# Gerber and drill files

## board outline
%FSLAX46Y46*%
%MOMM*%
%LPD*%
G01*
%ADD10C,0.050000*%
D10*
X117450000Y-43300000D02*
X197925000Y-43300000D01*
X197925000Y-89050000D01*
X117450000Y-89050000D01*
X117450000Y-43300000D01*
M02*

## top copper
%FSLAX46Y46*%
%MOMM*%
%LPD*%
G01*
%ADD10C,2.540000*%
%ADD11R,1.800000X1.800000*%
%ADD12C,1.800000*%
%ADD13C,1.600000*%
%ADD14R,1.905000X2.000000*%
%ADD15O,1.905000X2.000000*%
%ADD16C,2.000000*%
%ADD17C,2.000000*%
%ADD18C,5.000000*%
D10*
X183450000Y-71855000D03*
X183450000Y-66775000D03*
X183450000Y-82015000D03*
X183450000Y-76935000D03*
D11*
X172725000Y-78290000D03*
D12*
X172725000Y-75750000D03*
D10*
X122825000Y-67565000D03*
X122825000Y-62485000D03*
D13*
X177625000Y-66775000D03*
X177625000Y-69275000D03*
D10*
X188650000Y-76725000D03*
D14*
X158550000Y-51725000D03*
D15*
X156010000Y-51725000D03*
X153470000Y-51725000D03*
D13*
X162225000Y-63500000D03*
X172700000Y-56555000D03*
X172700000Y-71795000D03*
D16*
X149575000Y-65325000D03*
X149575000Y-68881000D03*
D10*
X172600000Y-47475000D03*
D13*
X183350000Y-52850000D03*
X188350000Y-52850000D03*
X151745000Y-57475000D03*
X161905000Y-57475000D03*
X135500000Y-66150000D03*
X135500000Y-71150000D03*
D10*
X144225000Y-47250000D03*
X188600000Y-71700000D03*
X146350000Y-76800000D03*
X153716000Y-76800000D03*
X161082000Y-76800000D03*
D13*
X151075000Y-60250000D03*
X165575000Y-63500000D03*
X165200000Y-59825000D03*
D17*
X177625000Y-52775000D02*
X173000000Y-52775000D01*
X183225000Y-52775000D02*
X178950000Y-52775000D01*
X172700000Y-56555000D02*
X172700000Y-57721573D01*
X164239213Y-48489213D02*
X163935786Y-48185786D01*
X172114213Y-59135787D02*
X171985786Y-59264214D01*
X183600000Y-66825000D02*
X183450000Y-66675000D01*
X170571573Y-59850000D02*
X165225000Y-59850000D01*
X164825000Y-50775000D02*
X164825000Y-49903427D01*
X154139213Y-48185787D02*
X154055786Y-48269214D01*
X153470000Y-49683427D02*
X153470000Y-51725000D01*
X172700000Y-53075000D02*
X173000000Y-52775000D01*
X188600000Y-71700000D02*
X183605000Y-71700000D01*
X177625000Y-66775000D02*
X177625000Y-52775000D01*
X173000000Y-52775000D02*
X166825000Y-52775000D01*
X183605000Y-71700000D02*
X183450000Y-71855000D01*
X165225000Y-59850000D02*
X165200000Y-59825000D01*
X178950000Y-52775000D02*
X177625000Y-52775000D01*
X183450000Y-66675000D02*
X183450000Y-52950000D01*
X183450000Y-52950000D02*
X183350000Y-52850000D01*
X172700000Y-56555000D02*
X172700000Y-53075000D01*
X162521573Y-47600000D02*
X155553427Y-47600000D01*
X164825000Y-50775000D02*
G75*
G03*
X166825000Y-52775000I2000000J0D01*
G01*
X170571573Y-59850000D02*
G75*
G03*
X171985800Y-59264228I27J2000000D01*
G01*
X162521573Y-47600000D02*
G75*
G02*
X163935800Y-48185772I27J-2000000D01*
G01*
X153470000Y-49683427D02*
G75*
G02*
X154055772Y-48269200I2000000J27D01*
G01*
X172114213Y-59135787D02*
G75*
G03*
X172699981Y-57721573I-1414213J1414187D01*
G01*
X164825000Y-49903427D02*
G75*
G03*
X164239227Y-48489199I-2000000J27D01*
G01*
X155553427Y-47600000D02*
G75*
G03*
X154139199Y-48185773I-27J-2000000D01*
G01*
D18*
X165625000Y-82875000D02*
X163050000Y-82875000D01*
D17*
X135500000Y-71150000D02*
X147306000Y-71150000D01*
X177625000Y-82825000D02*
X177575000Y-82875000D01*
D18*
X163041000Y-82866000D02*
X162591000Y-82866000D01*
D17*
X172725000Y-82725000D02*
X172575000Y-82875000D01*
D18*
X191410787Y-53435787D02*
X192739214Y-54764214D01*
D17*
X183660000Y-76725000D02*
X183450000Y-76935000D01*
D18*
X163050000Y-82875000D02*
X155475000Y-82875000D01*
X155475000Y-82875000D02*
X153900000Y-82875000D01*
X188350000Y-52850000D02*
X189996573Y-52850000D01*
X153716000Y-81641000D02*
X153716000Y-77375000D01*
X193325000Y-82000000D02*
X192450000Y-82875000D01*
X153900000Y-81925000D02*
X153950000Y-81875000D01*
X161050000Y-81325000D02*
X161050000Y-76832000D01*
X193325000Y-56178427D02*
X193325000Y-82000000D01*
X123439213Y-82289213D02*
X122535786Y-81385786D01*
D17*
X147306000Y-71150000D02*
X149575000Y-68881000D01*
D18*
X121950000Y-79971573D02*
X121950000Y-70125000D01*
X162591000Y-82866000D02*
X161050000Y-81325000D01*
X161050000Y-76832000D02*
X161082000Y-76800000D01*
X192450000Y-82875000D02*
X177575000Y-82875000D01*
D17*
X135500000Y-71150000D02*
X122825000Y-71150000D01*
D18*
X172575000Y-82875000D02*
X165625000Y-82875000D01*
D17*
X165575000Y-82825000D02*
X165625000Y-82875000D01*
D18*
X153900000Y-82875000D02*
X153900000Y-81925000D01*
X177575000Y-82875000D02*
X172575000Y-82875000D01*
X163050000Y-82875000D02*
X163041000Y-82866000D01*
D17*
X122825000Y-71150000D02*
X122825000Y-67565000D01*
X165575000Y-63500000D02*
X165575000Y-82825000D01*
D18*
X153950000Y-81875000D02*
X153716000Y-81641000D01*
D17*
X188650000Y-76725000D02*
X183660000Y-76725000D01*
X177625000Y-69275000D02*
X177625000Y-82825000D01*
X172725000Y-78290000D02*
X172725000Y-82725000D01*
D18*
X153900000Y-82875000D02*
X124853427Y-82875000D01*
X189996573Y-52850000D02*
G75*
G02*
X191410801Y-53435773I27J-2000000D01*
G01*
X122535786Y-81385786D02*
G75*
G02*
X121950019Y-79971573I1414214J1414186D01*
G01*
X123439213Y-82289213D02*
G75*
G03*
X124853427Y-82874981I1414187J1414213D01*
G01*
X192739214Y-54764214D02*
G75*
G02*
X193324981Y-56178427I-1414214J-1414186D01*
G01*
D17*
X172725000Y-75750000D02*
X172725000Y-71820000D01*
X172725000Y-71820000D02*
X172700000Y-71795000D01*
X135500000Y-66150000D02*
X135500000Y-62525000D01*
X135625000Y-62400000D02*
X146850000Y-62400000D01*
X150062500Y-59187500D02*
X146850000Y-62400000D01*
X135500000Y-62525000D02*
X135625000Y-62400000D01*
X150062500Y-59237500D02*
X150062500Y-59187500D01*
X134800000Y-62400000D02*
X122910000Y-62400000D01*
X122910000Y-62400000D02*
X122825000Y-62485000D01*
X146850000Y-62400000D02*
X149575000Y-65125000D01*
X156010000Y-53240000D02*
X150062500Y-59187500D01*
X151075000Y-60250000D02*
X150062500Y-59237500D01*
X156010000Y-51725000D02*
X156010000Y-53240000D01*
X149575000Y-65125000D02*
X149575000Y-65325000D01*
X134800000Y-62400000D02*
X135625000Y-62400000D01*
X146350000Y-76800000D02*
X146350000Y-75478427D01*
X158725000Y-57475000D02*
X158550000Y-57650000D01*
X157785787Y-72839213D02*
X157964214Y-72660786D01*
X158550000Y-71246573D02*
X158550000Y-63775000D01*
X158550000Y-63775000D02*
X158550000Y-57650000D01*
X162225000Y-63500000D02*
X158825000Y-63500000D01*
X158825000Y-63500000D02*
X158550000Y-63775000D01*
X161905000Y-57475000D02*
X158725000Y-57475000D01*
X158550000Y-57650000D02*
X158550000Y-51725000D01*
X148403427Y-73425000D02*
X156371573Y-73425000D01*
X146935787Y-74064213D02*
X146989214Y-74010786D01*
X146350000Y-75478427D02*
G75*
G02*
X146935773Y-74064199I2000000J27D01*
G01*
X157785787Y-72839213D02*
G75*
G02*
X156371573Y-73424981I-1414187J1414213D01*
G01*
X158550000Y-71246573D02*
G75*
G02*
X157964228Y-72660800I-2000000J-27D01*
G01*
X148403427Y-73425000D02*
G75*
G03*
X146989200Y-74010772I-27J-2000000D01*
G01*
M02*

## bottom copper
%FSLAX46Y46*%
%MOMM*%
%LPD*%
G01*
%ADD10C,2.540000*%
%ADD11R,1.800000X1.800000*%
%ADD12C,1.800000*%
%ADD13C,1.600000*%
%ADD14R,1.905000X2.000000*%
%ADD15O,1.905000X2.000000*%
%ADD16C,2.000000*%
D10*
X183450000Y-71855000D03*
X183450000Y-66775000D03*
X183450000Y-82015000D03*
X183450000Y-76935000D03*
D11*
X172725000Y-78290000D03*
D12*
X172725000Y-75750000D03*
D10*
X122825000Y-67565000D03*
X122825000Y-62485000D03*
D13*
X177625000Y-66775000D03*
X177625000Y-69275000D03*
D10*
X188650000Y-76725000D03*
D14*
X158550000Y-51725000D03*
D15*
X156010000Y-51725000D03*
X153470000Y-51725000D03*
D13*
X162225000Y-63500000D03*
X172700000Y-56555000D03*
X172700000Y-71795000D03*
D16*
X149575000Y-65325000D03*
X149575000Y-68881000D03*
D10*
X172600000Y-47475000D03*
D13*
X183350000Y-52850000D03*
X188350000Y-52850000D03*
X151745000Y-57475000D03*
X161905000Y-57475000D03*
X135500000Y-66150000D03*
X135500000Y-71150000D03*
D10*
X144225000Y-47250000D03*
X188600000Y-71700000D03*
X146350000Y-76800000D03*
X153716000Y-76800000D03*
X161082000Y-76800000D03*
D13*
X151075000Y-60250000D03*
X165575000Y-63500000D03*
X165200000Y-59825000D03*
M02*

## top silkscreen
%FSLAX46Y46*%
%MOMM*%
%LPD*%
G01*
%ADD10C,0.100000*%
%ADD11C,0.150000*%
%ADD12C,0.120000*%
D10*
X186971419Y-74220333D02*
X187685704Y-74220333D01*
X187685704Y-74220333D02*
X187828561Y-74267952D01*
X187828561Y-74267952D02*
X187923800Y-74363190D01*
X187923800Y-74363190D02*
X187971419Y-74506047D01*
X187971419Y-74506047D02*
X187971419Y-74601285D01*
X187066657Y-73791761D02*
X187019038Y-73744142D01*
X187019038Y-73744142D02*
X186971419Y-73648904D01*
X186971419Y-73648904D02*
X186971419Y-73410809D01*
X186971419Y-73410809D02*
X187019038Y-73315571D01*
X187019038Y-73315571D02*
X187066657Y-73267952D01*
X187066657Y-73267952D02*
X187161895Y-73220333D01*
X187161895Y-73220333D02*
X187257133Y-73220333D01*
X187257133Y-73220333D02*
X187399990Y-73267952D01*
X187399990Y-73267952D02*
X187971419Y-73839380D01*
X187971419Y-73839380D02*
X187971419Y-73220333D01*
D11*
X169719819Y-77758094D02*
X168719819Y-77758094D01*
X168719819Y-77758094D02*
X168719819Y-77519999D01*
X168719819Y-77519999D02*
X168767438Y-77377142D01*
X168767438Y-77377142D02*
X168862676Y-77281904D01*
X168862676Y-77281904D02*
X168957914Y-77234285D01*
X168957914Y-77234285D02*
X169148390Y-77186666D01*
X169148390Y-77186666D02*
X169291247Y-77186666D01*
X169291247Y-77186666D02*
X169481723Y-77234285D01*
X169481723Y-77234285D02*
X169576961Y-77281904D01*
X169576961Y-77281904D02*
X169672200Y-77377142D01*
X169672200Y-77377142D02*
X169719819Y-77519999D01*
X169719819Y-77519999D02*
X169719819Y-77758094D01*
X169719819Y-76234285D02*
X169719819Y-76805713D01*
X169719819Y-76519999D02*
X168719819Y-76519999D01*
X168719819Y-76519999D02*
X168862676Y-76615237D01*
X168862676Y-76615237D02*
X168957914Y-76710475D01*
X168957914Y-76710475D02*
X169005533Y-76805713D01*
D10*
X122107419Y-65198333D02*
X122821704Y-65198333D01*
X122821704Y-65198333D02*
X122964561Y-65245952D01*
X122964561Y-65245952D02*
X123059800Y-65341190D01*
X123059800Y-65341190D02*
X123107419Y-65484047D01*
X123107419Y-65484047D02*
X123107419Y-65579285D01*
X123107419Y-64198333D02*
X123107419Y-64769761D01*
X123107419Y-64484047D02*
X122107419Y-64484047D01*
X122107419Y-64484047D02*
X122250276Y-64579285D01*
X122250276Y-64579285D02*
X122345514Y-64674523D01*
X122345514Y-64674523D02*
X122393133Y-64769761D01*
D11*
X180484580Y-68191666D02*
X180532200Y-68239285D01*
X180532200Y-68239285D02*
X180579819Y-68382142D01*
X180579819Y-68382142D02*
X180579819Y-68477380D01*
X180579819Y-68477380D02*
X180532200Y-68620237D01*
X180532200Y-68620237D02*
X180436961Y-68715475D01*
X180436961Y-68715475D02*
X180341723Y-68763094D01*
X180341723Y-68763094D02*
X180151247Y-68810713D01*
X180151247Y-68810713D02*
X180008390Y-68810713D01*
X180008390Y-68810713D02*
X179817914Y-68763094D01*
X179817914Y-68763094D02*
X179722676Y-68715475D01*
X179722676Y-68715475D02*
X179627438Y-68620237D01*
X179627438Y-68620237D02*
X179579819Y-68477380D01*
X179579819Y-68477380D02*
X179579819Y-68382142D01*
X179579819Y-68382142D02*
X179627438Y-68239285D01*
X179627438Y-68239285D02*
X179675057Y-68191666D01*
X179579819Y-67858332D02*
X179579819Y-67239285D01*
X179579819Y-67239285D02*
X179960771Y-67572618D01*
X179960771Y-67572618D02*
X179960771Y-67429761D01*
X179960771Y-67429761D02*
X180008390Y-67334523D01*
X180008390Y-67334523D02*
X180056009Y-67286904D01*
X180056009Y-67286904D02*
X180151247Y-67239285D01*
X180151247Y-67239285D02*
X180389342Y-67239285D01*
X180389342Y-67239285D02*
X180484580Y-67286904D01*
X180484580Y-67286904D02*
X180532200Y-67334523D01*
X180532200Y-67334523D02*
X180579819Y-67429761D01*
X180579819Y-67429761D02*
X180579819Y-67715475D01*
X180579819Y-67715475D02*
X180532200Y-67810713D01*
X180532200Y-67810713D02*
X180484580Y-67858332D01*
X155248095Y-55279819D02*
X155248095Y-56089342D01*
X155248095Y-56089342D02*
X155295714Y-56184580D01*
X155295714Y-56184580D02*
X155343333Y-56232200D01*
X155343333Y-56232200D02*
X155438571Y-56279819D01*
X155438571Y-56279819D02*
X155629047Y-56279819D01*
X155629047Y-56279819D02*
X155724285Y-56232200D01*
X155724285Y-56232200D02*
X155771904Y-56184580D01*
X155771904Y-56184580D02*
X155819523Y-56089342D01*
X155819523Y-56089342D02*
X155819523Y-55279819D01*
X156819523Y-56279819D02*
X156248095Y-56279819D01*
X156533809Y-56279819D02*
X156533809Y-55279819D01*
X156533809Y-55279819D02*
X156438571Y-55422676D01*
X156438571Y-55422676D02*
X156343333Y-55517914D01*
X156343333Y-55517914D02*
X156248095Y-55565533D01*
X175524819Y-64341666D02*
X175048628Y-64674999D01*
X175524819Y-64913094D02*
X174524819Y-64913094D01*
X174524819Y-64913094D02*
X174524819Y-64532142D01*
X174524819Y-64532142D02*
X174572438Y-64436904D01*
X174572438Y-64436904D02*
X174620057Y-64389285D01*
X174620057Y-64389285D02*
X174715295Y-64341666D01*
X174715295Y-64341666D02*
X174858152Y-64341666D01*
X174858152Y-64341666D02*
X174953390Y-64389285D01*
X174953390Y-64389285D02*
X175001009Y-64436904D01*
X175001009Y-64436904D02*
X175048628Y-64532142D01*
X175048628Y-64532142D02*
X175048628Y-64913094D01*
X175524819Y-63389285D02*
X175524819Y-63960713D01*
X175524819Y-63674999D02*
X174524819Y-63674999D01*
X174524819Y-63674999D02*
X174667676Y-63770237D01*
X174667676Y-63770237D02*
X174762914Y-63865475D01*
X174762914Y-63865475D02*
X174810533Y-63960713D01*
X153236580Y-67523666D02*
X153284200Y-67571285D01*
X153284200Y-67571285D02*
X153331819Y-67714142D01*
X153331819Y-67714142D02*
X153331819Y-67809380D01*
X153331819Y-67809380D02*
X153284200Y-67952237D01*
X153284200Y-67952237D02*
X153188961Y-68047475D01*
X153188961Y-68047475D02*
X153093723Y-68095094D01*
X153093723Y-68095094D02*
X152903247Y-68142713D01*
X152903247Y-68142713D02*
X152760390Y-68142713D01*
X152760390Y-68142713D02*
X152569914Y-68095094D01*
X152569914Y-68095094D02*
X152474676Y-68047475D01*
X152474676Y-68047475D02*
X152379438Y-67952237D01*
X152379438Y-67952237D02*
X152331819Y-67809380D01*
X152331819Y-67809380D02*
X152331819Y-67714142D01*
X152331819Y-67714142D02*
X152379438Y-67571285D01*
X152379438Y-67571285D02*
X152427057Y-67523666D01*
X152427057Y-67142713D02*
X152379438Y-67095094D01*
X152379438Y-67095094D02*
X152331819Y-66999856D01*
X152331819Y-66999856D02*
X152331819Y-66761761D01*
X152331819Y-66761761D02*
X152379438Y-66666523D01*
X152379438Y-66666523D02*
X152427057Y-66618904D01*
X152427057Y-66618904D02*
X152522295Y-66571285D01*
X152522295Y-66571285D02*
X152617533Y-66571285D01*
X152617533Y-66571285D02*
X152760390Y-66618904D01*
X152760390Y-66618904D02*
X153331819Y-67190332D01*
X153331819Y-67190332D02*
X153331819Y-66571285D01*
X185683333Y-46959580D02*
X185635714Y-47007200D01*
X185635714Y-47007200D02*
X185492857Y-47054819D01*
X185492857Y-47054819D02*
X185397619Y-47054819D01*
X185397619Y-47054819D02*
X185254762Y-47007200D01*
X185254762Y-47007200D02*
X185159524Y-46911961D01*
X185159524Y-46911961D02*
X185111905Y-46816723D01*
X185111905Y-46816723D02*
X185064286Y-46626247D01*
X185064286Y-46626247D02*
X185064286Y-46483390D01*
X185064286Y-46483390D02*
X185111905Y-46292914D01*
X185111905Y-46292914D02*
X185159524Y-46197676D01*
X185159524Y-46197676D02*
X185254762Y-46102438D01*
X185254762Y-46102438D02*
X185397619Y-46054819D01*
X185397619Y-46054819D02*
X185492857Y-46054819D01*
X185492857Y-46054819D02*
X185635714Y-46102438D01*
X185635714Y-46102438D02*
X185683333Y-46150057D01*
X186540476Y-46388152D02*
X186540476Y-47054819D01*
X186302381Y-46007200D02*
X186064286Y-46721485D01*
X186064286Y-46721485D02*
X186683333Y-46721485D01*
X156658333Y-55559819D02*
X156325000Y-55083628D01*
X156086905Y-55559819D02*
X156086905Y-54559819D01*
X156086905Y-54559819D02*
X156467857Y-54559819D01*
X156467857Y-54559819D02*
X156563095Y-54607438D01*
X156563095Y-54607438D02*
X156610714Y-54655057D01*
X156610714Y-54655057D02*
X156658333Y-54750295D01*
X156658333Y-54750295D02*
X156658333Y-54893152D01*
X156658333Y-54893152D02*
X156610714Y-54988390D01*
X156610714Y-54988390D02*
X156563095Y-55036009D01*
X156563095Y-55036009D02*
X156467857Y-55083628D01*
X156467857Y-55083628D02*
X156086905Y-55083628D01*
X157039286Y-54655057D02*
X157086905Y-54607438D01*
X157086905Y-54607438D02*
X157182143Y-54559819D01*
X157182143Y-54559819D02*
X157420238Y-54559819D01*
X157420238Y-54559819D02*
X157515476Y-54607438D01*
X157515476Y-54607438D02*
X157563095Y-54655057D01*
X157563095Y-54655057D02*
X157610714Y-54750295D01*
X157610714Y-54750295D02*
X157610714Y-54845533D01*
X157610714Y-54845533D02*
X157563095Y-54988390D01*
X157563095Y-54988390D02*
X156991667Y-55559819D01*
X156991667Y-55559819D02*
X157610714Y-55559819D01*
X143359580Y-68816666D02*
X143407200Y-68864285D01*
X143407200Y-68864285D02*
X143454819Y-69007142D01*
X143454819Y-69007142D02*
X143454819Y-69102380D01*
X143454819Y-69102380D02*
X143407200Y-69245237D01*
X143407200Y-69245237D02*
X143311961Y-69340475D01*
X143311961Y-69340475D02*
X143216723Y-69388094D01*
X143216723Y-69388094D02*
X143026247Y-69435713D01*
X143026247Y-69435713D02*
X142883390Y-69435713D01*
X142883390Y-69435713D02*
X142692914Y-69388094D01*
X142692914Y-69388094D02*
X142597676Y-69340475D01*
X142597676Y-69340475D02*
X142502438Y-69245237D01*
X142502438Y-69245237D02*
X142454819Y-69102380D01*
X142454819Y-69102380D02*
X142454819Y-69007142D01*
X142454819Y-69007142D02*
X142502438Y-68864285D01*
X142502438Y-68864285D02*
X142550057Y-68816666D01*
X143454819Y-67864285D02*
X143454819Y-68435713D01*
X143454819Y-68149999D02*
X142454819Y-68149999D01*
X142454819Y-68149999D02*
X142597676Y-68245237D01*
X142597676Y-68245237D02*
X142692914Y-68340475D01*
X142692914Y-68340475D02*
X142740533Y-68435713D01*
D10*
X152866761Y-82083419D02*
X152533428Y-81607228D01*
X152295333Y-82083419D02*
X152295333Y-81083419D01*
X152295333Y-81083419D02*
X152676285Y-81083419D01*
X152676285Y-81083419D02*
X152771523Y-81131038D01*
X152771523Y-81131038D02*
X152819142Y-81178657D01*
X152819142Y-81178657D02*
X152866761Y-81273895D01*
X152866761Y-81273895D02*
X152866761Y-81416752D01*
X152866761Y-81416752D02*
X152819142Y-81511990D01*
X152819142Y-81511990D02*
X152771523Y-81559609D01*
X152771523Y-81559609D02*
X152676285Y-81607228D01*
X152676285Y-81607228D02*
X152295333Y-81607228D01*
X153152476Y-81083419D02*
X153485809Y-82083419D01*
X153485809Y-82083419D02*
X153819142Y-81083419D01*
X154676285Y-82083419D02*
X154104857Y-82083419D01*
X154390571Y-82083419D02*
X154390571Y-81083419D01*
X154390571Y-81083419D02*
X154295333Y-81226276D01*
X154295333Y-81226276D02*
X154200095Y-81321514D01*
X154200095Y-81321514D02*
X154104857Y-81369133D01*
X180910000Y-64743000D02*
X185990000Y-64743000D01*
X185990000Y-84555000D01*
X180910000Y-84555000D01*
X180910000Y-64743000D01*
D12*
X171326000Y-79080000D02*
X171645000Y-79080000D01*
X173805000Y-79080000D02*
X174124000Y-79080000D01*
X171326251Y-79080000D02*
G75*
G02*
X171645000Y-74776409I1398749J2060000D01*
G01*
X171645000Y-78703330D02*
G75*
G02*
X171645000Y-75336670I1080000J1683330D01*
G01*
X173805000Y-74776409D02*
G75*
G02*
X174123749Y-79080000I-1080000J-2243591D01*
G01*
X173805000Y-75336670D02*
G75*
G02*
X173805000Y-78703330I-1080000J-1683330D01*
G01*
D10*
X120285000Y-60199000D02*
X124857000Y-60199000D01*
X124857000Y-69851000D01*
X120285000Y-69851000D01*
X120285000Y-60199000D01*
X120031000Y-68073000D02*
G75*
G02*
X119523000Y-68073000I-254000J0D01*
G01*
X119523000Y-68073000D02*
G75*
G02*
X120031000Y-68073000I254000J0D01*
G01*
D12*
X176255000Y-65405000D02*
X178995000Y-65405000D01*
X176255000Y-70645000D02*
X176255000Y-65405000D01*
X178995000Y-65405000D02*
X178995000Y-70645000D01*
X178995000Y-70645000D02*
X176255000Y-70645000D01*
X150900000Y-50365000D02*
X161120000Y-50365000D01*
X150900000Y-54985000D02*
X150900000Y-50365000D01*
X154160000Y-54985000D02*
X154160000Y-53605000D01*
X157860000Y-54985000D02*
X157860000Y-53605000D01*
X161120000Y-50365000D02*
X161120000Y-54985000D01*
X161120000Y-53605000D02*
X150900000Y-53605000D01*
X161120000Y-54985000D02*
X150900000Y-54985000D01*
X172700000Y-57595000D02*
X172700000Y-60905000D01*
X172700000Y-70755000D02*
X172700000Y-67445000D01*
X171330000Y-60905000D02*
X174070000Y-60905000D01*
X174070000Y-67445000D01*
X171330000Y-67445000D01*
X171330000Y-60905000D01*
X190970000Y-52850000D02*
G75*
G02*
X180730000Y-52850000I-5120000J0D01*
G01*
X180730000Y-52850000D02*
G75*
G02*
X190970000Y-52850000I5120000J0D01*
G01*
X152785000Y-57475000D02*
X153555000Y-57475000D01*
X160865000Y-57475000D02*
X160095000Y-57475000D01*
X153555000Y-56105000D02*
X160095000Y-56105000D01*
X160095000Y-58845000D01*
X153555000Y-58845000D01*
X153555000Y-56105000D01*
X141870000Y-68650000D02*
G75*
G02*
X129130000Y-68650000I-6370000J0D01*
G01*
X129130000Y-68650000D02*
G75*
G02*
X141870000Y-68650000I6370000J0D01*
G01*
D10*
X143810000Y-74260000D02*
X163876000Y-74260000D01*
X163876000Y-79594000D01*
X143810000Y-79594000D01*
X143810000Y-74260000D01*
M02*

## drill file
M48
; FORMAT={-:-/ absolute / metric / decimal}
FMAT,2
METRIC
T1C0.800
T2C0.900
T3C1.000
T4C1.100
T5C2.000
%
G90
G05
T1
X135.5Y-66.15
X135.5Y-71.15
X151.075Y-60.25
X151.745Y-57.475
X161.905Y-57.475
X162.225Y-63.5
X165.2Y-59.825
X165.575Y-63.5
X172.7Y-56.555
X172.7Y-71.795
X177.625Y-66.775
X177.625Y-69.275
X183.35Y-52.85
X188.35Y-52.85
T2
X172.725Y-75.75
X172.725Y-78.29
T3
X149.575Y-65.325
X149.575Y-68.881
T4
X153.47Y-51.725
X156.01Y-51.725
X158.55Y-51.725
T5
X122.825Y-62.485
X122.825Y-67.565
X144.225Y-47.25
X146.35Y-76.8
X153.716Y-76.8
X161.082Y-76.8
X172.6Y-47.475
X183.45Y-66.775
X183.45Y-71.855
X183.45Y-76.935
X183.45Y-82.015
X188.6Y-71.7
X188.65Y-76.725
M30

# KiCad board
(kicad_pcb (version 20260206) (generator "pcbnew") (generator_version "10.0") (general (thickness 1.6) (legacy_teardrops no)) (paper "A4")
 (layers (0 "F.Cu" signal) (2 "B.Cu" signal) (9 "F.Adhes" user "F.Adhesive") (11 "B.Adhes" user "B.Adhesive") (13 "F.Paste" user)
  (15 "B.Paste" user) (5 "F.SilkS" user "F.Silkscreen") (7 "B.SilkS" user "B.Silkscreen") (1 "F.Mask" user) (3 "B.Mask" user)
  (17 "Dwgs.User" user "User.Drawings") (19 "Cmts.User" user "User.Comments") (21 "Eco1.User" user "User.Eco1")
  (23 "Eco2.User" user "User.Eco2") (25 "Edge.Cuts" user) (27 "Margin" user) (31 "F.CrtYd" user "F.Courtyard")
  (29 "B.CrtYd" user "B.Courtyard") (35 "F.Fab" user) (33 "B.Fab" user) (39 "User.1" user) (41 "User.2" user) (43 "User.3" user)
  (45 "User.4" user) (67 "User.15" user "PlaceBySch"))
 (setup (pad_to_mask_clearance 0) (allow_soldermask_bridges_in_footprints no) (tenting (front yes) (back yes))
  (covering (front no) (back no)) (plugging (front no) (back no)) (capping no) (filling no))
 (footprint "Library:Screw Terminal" (layer "F.Cu") (at 183.45 74.395 90)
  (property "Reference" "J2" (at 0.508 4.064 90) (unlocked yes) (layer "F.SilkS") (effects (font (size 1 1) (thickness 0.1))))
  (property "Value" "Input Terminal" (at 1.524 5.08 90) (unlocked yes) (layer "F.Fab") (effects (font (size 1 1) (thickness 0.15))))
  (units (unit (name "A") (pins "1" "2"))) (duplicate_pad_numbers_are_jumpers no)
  (fp_rect (start -10.16 -2.54) (end 9.652 2.54) (stroke (width 0.1) (type default)) (fill no) (layer "F.SilkS"))
  (pad "1" thru_hole circle (at 2.54 0 90) (size 2.54 2.54) (drill 2) (layers "*.Cu" "*.Mask") (remove_unused_layers no)
   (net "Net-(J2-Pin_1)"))
  (pad "1" thru_hole circle (at 7.62 0 90) (size 2.54 2.54) (drill 2) (layers "*.Cu" "*.Mask") (remove_unused_layers no)
   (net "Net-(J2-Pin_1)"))
  (pad "2" thru_hole circle (at -7.62 0 90) (size 2.54 2.54) (drill 2) (layers "*.Cu" "*.Mask") (remove_unused_layers no) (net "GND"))
  (pad "2" thru_hole circle (at -2.54 0 90) (size 2.54 2.54) (drill 2) (layers "*.Cu" "*.Mask") (remove_unused_layers no) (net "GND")))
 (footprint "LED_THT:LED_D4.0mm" (layer "F.Cu") (at 172.725 78.29 90)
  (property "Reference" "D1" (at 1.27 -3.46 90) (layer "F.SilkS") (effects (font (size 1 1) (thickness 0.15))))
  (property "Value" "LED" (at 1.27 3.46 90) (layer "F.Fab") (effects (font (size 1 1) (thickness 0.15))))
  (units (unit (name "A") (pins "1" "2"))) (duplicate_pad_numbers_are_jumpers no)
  (fp_line (start -0.79 -1.399) (end -0.79 -1.08) (stroke (width 0.12) (type solid)) (layer "F.SilkS"))
  (fp_line (start -0.79 1.08) (end -0.79 1.399) (stroke (width 0.12) (type solid)) (layer "F.SilkS"))
  (fp_arc (start -0.79 -1.398749) (mid 1.45392 -2.483198) (end 3.513591 -1.08) (stroke (width 0.12) (type solid)) (layer "F.SilkS"))
  (fp_arc (start -0.41333 -1.08) (mid 1.27 -2) (end 2.95333 -1.08) (stroke (width 0.12) (type solid)) (layer "F.SilkS"))
  (fp_arc (start 3.513591 1.08) (mid 1.45392 2.483198) (end -0.79 1.398749) (stroke (width 0.12) (type solid)) (layer "F.SilkS"))
  (fp_arc (start 2.95333 1.08) (mid 1.27 2) (end -0.41333 1.08) (stroke (width 0.12) (type solid)) (layer "F.SilkS"))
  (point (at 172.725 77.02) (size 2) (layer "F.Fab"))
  (pad "1" thru_hole rect (at 0 0 90) (size 1.8 1.8) (drill 0.9) (layers "*.Cu" "*.Mask") (remove_unused_layers no) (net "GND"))
  (pad "2" thru_hole circle (at 2.54 0 90) (size 1.8 1.8) (drill 0.9) (layers "*.Cu" "*.Mask") (remove_unused_layers no) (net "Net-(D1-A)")))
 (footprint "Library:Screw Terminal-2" (layer "F.Cu") (at 122.825 65.025 90)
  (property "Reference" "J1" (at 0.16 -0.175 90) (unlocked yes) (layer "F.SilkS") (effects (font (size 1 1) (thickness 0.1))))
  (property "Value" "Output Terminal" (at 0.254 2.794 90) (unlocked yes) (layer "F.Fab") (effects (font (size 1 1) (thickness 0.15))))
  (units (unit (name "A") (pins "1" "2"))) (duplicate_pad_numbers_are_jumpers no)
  (fp_rect (start -4.826 -2.54) (end 4.826 2.032) (stroke (width 0.1) (type default)) (fill no) (layer "F.SilkS"))
  (fp_circle (center -3.048 -3.048) (end -2.794 -3.048) (stroke (width 0.1) (type solid)) (fill no) (layer "F.SilkS"))
  (pad "1" thru_hole circle (at -2.54 0 90) (size 2.54 2.54) (drill 2) (layers "*.Cu" "*.Mask") (remove_unused_layers no) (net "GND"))
  (pad "2" thru_hole circle (at 2.54 0 180) (size 2.54 2.54) (drill 2) (layers "*.Cu" "*.Mask") (remove_unused_layers no)
   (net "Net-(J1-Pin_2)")))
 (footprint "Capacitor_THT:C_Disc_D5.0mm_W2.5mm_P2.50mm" (layer "F.Cu") (at 177.625 66.775 -90)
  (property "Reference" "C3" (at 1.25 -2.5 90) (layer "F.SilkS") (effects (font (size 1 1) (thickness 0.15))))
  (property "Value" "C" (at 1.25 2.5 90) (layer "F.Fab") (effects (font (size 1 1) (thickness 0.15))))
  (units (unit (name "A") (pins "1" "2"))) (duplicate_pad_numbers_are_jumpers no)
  (fp_line (start -1.37 1.37) (end -1.37 -1.37) (stroke (width 0.12) (type solid)) (layer "F.SilkS"))
  (fp_line (start 3.87 1.37) (end -1.37 1.37) (stroke (width 0.12) (type solid)) (layer "F.SilkS"))
  (fp_line (start -1.37 -1.37) (end 3.87 -1.37) (stroke (width 0.12) (type solid)) (layer "F.SilkS"))
  (fp_line (start 3.87 -1.37) (end 3.87 1.37) (stroke (width 0.12) (type solid)) (layer "F.SilkS"))
  (pad "1" thru_hole circle (at 0 0 270) (size 1.6 1.6) (drill 0.8) (layers "*.Cu" "*.Mask") (remove_unused_layers no)
   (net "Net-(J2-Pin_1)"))
  (pad "2" thru_hole circle (at 2.5 0 270) (size 1.6 1.6) (drill 0.8) (layers "*.Cu" "*.Mask") (remove_unused_layers no) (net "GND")))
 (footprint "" (layer "F.Cu") (at 188.65 76.725)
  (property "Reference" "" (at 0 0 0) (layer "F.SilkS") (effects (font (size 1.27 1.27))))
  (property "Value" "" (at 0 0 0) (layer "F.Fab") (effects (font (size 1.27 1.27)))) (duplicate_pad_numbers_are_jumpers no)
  (pad "2" thru_hole circle (at 0 0 90) (size 2.54 2.54) (drill 2) (layers "*.Cu" "*.Mask") (remove_unused_layers no) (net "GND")))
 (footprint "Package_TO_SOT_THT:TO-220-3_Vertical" (layer "F.Cu") (at 158.55 51.725 180)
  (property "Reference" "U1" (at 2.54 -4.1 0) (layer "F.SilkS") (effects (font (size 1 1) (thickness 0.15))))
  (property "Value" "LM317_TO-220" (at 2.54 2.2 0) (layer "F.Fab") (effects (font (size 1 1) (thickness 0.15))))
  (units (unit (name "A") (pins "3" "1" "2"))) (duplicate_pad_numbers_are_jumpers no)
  (fp_line (start 7.65 1.36) (end -2.57 1.36) (stroke (width 0.12) (type solid)) (layer "F.SilkS"))
  (fp_line (start 7.65 -3.26) (end 7.65 1.36) (stroke (width 0.12) (type solid)) (layer "F.SilkS"))
  (fp_line (start 4.39 -3.26) (end 4.39 -1.88) (stroke (width 0.12) (type solid)) (layer "F.SilkS"))
  (fp_line (start 0.69 -3.26) (end 0.69 -1.88) (stroke (width 0.12) (type solid)) (layer "F.SilkS"))
  (fp_line (start -2.57 1.36) (end -2.57 -3.26) (stroke (width 0.12) (type solid)) (layer "F.SilkS"))
  (fp_line (start -2.57 -1.88) (end 7.65 -1.88) (stroke (width 0.12) (type solid)) (layer "F.SilkS"))
  (fp_line (start -2.57 -3.26) (end 7.65 -3.26) (stroke (width 0.12) (type solid)) (layer "F.SilkS"))
  (pad "1" thru_hole rect (at 0 0 180) (size 1.905 2) (drill 1.1) (layers "*.Cu" "*.Mask") (remove_unused_layers no) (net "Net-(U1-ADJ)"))
  (pad "2" thru_hole oval (at 2.54 0 180) (size 1.905 2) (drill 1.1) (layers "*.Cu" "*.Mask") (remove_unused_layers no)
   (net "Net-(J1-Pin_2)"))
  (pad "3" thru_hole oval (at 5.08 0 180) (size 1.905 2) (drill 1.1) (layers "*.Cu" "*.Mask") (remove_unused_layers no)
   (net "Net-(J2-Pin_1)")))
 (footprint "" (layer "F.Cu") (at 162.225 63.5)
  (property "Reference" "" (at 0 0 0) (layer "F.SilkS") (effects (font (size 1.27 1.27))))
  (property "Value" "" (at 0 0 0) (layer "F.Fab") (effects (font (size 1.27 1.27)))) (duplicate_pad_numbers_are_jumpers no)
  (pad "2" thru_hole circle (at 0 0) (size 1.6 1.6) (drill 0.8) (layers "*.Cu" "*.Mask") (remove_unused_layers no) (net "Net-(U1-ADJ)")))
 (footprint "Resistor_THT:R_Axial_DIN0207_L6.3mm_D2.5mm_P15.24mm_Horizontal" (layer "F.Cu") (at 172.7 56.555 -90)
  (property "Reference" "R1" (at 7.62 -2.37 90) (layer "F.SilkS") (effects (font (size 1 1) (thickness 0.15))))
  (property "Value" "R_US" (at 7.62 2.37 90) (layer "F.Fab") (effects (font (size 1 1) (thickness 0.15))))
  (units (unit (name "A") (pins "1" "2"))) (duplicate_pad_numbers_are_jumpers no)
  (fp_line (start 1.04 0) (end 4.35 0) (stroke (width 0.12) (type solid)) (layer "F.SilkS"))
  (fp_line (start 14.2 0) (end 10.89 0) (stroke (width 0.12) (type solid)) (layer "F.SilkS"))
  (fp_rect (start 4.35 -1.37) (end 10.89 1.37) (stroke (width 0.12) (type solid)) (fill no) (layer "F.SilkS"))
  (pad "1" thru_hole circle (at 0 0 270) (size 1.6 1.6) (drill 0.8) (layers "*.Cu" "*.Mask") (remove_unused_layers no)
   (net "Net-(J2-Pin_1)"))
  (pad "2" thru_hole circle (at 15.24 0 270) (size 1.6 1.6) (drill 0.8) (layers "*.Cu" "*.Mask") (remove_unused_layers no)
   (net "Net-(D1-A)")))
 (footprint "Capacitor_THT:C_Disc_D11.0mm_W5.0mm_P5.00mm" (layer "F.Cu") (at 149.575 65.325 -90)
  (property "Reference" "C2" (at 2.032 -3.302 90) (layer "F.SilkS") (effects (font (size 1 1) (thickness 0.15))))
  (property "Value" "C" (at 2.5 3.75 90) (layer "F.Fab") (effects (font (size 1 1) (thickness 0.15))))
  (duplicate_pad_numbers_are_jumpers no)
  (pad "1" thru_hole circle (at 0 0 270) (size 2 2) (drill 1) (layers "*.Cu" "*.Mask") (remove_unused_layers no) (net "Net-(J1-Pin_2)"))
  (pad "2" thru_hole circle (at 3.556 0 270) (size 2 2) (drill 1) (layers "*.Cu" "*.Mask") (remove_unused_layers no) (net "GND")))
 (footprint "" (layer "F.Cu") (at 172.6 47.475)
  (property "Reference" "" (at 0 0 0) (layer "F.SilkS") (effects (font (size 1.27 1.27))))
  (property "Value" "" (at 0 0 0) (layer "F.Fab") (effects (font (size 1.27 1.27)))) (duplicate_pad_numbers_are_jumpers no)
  (pad "3" thru_hole circle (at 0 0) (size 2.54 2.54) (drill 2) (layers "*.Cu" "*.Mask") (remove_unused_layers no) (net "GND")))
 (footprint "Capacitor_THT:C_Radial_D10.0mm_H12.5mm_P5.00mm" (layer "F.Cu") (at 183.35 52.85)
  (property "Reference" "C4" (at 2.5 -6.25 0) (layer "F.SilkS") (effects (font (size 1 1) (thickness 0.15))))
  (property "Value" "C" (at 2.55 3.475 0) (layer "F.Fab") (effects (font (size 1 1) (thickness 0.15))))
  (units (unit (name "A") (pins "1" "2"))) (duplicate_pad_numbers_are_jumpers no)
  (fp_circle (center 2.5 0) (end 7.62 0) (stroke (width 0.12) (type solid)) (fill no) (layer "F.SilkS"))
  (pad "1" thru_hole circle (at 0 0) (size 1.6 1.6) (drill 0.8) (layers "*.Cu" "*.Mask") (remove_unused_layers no) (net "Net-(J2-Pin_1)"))
  (pad "2" thru_hole circle (at 5 0) (size 1.6 1.6) (drill 0.8) (layers "*.Cu" "*.Mask") (remove_unused_layers no) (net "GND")))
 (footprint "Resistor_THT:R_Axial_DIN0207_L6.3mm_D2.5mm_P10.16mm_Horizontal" (layer "F.Cu") (at 151.745 57.475)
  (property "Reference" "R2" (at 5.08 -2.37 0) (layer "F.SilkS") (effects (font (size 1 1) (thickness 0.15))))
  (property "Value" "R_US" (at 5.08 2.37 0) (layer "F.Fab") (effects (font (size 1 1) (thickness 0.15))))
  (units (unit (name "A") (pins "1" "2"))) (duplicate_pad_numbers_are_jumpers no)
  (fp_line (start 1.04 0) (end 1.81 0) (stroke (width 0.12) (type solid)) (layer "F.SilkS"))
  (fp_line (start 9.12 0) (end 8.35 0) (stroke (width 0.12) (type solid)) (layer "F.SilkS"))
  (fp_rect (start 1.81 -1.37) (end 8.35 1.37) (stroke (width 0.12) (type solid)) (fill no) (layer "F.SilkS"))
  (pad "1" thru_hole circle (at 0 0) (size 1.6 1.6) (drill 0.8) (layers "*.Cu" "*.Mask") (remove_unused_layers no) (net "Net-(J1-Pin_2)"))
  (pad "2" thru_hole circle (at 10.16 0) (size 1.6 1.6) (drill 0.8) (layers "*.Cu" "*.Mask") (remove_unused_layers no) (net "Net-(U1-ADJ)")))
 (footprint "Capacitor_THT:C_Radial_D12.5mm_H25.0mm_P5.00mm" (layer "F.Cu") (at 135.5 66.15 -90)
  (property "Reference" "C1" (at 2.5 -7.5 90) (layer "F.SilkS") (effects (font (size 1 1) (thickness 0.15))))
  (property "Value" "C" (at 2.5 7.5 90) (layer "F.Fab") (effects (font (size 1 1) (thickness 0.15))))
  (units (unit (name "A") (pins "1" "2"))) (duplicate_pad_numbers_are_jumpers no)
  (fp_circle (center 2.5 0) (end 8.87 0) (stroke (width 0.12) (type solid)) (fill no) (layer "F.SilkS"))
  (pad "1" thru_hole circle (at 0 0 270) (size 1.6 1.6) (drill 0.8) (layers "*.Cu" "*.Mask") (remove_unused_layers no)
   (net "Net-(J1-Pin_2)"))
  (pad "2" thru_hole circle (at 5 0 270) (size 1.6 1.6) (drill 0.8) (layers "*.Cu" "*.Mask") (remove_unused_layers no) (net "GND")))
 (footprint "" (layer "F.Cu") (at 144.225 47.25)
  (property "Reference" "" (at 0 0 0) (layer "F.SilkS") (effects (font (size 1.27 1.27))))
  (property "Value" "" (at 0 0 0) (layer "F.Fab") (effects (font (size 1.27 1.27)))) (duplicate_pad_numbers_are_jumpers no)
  (pad "3" thru_hole circle (at 0 0) (size 2.54 2.54) (drill 2) (layers "*.Cu" "*.Mask") (remove_unused_layers no) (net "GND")))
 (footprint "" (layer "F.Cu") (at 188.6 71.7)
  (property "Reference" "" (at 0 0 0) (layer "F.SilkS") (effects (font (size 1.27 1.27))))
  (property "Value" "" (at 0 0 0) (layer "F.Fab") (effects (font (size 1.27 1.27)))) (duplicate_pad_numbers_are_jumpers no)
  (pad "1" thru_hole circle (at 0 0 90) (size 2.54 2.54) (drill 2) (layers "*.Cu" "*.Mask") (remove_unused_layers no) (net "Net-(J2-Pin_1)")))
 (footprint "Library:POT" (layer "F.Cu") (at 153.716 76.8)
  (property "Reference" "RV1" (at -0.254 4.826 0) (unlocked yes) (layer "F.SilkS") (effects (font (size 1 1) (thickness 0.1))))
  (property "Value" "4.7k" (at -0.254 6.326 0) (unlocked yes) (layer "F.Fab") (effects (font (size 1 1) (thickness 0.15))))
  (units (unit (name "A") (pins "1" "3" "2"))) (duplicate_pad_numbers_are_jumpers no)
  (fp_rect (start -9.906 -2.54) (end 10.16 2.794) (stroke (width 0.1) (type default)) (fill no) (layer "F.SilkS"))
  (pad "1" thru_hole circle (at -7.366 0) (size 2.54 2.54) (drill 2) (layers "*.Cu" "*.Mask") (remove_unused_layers no) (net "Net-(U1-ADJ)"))
  (pad "2" thru_hole circle (at 0 0) (size 2.54 2.54) (drill 2) (layers "*.Cu" "*.Mask") (remove_unused_layers no) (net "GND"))
  (pad "3" thru_hole circle (at 7.366 0) (size 2.54 2.54) (drill 2) (layers "*.Cu" "*.Mask") (remove_unused_layers no) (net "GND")))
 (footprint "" (layer "F.Cu") (at 151.075 60.25)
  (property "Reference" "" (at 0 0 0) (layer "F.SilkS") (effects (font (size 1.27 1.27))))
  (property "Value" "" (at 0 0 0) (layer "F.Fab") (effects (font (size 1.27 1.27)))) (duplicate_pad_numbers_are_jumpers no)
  (pad "1" thru_hole circle (at 0 0) (size 1.6 1.6) (drill 0.8) (layers "*.Cu" "*.Mask") (remove_unused_layers no) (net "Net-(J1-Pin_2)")))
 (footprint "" (layer "F.Cu") (at 165.575 63.5)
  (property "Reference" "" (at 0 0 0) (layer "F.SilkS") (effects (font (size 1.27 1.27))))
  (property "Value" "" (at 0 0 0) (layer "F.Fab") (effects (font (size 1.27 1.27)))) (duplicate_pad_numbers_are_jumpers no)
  (pad "2" thru_hole circle (at 0 0) (size 1.6 1.6) (drill 0.8) (layers "*.Cu" "*.Mask") (remove_unused_layers no) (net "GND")))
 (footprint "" (layer "F.Cu") (at 165.2 59.825)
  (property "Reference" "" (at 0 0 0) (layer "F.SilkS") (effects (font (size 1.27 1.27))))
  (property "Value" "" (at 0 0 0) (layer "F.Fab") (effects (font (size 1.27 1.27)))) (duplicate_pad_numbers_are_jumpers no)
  (pad "1" thru_hole circle (at 0 0) (size 1.6 1.6) (drill 0.8) (layers "*.Cu" "*.Mask") (remove_unused_layers no) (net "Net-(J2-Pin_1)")))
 (gr_rect (start 117.45 43.3) (end 197.925 89.05) (stroke (width 0.05) (type default)) (fill no) (layer "Edge.Cuts"))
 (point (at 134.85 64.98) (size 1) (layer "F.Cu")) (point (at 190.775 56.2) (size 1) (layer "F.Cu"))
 (segment (start 177.625 52.775) (end 173 52.775) (width 2) (layer "F.Cu") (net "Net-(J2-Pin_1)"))
 (segment (start 183.225 52.775) (end 178.95 52.775) (width 2) (layer "F.Cu") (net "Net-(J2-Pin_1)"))
 (segment (start 172.7 56.555) (end 172.7 57.721573) (width 2) (layer "F.Cu") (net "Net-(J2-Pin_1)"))
 (segment (start 164.239213 48.489213) (end 163.935786 48.185786) (width 2) (layer "F.Cu") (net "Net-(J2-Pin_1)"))
 (segment (start 172.114213 59.135787) (end 171.985786 59.264214) (width 2) (layer "F.Cu") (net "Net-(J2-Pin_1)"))
 (segment (start 183.6 66.825) (end 183.45 66.675) (width 2) (layer "F.Cu") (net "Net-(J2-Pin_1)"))
 (segment (start 170.571573 59.85) (end 165.225 59.85) (width 2) (layer "F.Cu") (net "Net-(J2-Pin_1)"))
 (segment (start 164.825 50.775) (end 164.825 49.903427) (width 2) (layer "F.Cu") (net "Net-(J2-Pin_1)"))
 (segment (start 154.139213 48.185787) (end 154.055786 48.269214) (width 2) (layer "F.Cu") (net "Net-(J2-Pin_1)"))
 (segment (start 153.47 49.683427) (end 153.47 51.725) (width 2) (layer "F.Cu") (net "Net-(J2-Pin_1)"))
 (segment (start 172.7 53.075) (end 173 52.775) (width 2) (layer "F.Cu") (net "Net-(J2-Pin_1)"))
 (segment (start 188.6 71.7) (end 183.605 71.7) (width 2) (layer "F.Cu") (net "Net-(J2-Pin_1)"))
 (segment (start 177.625 66.775) (end 177.625 52.775) (width 2) (layer "F.Cu") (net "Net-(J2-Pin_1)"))
 (segment (start 173 52.775) (end 166.825 52.775) (width 2) (layer "F.Cu") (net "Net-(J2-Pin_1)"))
 (segment (start 183.605 71.7) (end 183.45 71.855) (width 2) (layer "F.Cu") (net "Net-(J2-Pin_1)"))
 (segment (start 165.225 59.85) (end 165.2 59.825) (width 2) (layer "F.Cu") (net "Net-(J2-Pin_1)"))
 (segment (start 178.95 52.775) (end 177.625 52.775) (width 2) (layer "F.Cu") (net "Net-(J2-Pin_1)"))
 (segment (start 183.45 66.675) (end 183.45 52.95) (width 2) (layer "F.Cu") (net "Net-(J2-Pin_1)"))
 (segment (start 183.45 52.95) (end 183.35 52.85) (width 2) (layer "F.Cu") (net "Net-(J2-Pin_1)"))
 (segment (start 172.7 56.555) (end 172.7 53.075) (width 2) (layer "F.Cu") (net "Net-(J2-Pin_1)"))
 (segment (start 162.521573 47.6) (end 155.553427 47.6) (width 2) (layer "F.Cu") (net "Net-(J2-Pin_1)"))
 (arc (start 164.825 50.775) (mid 165.410786 52.189214) (end 166.825 52.775) (width 2) (layer "F.Cu") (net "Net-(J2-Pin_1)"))
 (arc (start 170.571573 59.85) (mid 171.33694 59.697759) (end 171.985786 59.264214) (width 2) (layer "F.Cu") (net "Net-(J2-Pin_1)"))
 (arc (start 162.521573 47.6) (mid 163.28694 47.752241) (end 163.935786 48.185786) (width 2) (layer "F.Cu") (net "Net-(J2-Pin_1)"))
 (arc (start 153.47 49.683427) (mid 153.622241 48.91806) (end 154.055786 48.269214) (width 2) (layer "F.Cu") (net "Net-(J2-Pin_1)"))
 (arc (start 172.114213 59.135787) (mid 172.547759 58.48694) (end 172.7 57.721573) (width 2) (layer "F.Cu") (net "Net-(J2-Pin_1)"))
 (arc (start 164.825 49.903427) (mid 164.672759 49.13806) (end 164.239213 48.489213) (width 2) (layer "F.Cu") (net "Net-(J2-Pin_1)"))
 (arc (start 155.553427 47.6) (mid 154.78806 47.752241) (end 154.139213 48.185787) (width 2) (layer "F.Cu") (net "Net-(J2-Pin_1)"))
 (segment (start 165.625 82.875) (end 163.05 82.875) (width 5) (layer "F.Cu") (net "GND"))
 (segment (start 135.5 71.15) (end 147.306 71.15) (width 2) (layer "F.Cu") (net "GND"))
 (segment (start 177.625 82.825) (end 177.575 82.875) (width 2) (layer "F.Cu") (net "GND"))
 (segment (start 163.041 82.866) (end 162.591 82.866) (width 5) (layer "F.Cu") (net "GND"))
 (segment (start 172.725 82.725) (end 172.575 82.875) (width 2) (layer "F.Cu") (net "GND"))
 (segment (start 191.410787 53.435787) (end 192.739214 54.764214) (width 5) (layer "F.Cu") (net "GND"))
 (segment (start 183.66 76.725) (end 183.45 76.935) (width 2) (layer "F.Cu") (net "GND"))
 (segment (start 163.05 82.875) (end 155.475 82.875) (width 5) (layer "F.Cu") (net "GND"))
 (segment (start 155.475 82.875) (end 153.9 82.875) (width 5) (layer "F.Cu") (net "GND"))
 (segment (start 188.35 52.85) (end 189.996573 52.85) (width 5) (layer "F.Cu") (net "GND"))
 (segment (start 153.716 81.641) (end 153.716 77.375) (width 5) (layer "F.Cu") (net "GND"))
 (segment (start 193.325 82) (end 192.45 82.875) (width 5) (layer "F.Cu") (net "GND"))
 (segment (start 153.9 81.925) (end 153.95 81.875) (width 5) (layer "F.Cu") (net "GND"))
 (segment (start 161.05 81.325) (end 161.05 76.832) (width 5) (layer "F.Cu") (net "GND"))
 (segment (start 193.325 56.178427) (end 193.325 82) (width 5) (layer "F.Cu") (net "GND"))
 (segment (start 123.439213 82.289213) (end 122.535786 81.385786) (width 5) (layer "F.Cu") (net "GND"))
 (segment (start 147.306 71.15) (end 149.575 68.881) (width 2) (layer "F.Cu") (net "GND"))
 (segment (start 121.95 79.971573) (end 121.95 70.125) (width 5) (layer "F.Cu") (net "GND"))
 (segment (start 162.591 82.866) (end 161.05 81.325) (width 5) (layer "F.Cu") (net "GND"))
 (segment (start 161.05 76.832) (end 161.082 76.8) (width 5) (layer "F.Cu") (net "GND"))
 (segment (start 192.45 82.875) (end 177.575 82.875) (width 5) (layer "F.Cu") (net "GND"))
 (segment (start 135.5 71.15) (end 122.825 71.15) (width 2) (layer "F.Cu") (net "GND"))
 (segment (start 172.575 82.875) (end 165.625 82.875) (width 5) (layer "F.Cu") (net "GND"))
 (segment (start 165.575 82.825) (end 165.625 82.875) (width 2) (layer "F.Cu") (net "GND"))
 (segment (start 153.9 82.875) (end 153.9 81.925) (width 5) (layer "F.Cu") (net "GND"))
 (segment (start 177.575 82.875) (end 172.575 82.875) (width 5) (layer "F.Cu") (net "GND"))
 (segment (start 163.05 82.875) (end 163.041 82.866) (width 5) (layer "F.Cu") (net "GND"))
 (segment (start 122.825 71.15) (end 122.825 67.565) (width 2) (layer "F.Cu") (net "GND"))
 (segment (start 165.575 63.5) (end 165.575 82.825) (width 2) (layer "F.Cu") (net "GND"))
 (segment (start 153.95 81.875) (end 153.716 81.641) (width 5) (layer "F.Cu") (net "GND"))
 (segment (start 188.65 76.725) (end 183.66 76.725) (width 2) (layer "F.Cu") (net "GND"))
 (segment (start 177.625 69.275) (end 177.625 82.825) (width 2) (layer "F.Cu") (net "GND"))
 (segment (start 172.725 78.29) (end 172.725 82.725) (width 2) (layer "F.Cu") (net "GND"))
 (segment (start 153.9 82.875) (end 124.853427 82.875) (width 5) (layer "F.Cu") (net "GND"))
 (arc (start 189.996573 52.85) (mid 190.76194 53.002241) (end 191.410787 53.435787) (width 5) (layer "F.Cu") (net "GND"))
 (arc (start 122.535786 81.385786) (mid 122.102241 80.73694) (end 121.95 79.971573) (width 5) (layer "F.Cu") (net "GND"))
 (arc (start 123.439213 82.289213) (mid 124.08806 82.722759) (end 124.853427 82.875) (width 5) (layer "F.Cu") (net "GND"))
 (arc (start 192.739214 54.764214) (mid 193.172759 55.41306) (end 193.325 56.178427) (width 5) (layer "F.Cu") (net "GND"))
 (segment (start 172.725 75.75) (end 172.725 71.82) (width 2) (layer "F.Cu") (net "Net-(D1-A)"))
 (segment (start 172.725 71.82) (end 172.7 71.795) (width 2) (layer "F.Cu") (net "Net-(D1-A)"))
 (segment (start 135.5 66.15) (end 135.5 62.525) (width 2) (layer "F.Cu") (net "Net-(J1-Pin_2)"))
 (segment (start 135.625 62.4) (end 146.85 62.4) (width 2) (layer "F.Cu") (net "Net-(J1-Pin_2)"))
 (segment (start 150.0625 59.1875) (end 146.85 62.4) (width 2) (layer "F.Cu") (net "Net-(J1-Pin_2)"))
 (segment (start 135.5 62.525) (end 135.625 62.4) (width 2) (layer "F.Cu") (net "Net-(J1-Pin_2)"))
 (segment (start 150.0625 59.2375) (end 150.0625 59.1875) (width 2) (layer "F.Cu") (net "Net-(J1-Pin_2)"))
 (segment (start 134.8 62.4) (end 122.91 62.4) (width 2) (layer "F.Cu") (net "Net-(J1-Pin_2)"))
 (segment (start 122.91 62.4) (end 122.825 62.485) (width 2) (layer "F.Cu") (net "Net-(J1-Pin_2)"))
 (segment (start 146.85 62.4) (end 149.575 65.125) (width 2) (layer "F.Cu") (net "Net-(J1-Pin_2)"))
 (segment (start 156.01 53.24) (end 150.0625 59.1875) (width 2) (layer "F.Cu") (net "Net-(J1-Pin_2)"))
 (segment (start 151.075 60.25) (end 150.0625 59.2375) (width 2) (layer "F.Cu") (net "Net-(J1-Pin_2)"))
 (segment (start 156.01 51.725) (end 156.01 53.24) (width 2) (layer "F.Cu") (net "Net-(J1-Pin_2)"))
 (segment (start 149.575 65.125) (end 149.575 65.325) (width 2) (layer "F.Cu") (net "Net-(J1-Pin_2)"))
 (segment (start 134.8 62.4) (end 135.625 62.4) (width 2) (layer "F.Cu") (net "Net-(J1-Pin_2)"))
 (segment (start 146.35 76.8) (end 146.35 75.478427) (width 2) (layer "F.Cu") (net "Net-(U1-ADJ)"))
 (segment (start 158.725 57.475) (end 158.55 57.65) (width 2) (layer "F.Cu") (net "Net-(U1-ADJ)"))
 (segment (start 157.785787 72.839213) (end 157.964214 72.660786) (width 2) (layer "F.Cu") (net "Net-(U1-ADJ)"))
 (segment (start 158.55 71.246573) (end 158.55 63.775) (width 2) (layer "F.Cu") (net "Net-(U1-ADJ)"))
 (segment (start 158.55 63.775) (end 158.55 57.65) (width 2) (layer "F.Cu") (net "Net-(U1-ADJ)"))
 (segment (start 162.225 63.5) (end 158.825 63.5) (width 2) (layer "F.Cu") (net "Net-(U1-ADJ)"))
 (segment (start 158.825 63.5) (end 158.55 63.775) (width 2) (layer "F.Cu") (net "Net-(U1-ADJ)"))
 (segment (start 161.905 57.475) (end 158.725 57.475) (width 2) (layer "F.Cu") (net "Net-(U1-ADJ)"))
 (segment (start 158.55 57.65) (end 158.55 51.725) (width 2) (layer "F.Cu") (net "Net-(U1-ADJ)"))
 (segment (start 148.403427 73.425) (end 156.371573 73.425) (width 2) (layer "F.Cu") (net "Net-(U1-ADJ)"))
 (segment (start 146.935787 74.064213) (end 146.989214 74.010786) (width 2) (layer "F.Cu") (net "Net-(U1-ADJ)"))
 (arc (start 146.35 75.478427) (mid 146.502241 74.71306) (end 146.935787 74.064213) (width 2) (layer "F.Cu") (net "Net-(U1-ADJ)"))
 (arc (start 157.785787 72.839213) (mid 157.13694 73.272759) (end 156.371573 73.425) (width 2) (layer "F.Cu") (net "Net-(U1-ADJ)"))
 (arc (start 158.55 71.246573) (mid 158.397759 72.01194) (end 157.964214 72.660786) (width 2) (layer "F.Cu") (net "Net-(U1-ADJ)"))
 (arc (start 148.403427 73.425) (mid 147.63806 73.577241) (end 146.989214 74.010786) (width 2) (layer "F.Cu") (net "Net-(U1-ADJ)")))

